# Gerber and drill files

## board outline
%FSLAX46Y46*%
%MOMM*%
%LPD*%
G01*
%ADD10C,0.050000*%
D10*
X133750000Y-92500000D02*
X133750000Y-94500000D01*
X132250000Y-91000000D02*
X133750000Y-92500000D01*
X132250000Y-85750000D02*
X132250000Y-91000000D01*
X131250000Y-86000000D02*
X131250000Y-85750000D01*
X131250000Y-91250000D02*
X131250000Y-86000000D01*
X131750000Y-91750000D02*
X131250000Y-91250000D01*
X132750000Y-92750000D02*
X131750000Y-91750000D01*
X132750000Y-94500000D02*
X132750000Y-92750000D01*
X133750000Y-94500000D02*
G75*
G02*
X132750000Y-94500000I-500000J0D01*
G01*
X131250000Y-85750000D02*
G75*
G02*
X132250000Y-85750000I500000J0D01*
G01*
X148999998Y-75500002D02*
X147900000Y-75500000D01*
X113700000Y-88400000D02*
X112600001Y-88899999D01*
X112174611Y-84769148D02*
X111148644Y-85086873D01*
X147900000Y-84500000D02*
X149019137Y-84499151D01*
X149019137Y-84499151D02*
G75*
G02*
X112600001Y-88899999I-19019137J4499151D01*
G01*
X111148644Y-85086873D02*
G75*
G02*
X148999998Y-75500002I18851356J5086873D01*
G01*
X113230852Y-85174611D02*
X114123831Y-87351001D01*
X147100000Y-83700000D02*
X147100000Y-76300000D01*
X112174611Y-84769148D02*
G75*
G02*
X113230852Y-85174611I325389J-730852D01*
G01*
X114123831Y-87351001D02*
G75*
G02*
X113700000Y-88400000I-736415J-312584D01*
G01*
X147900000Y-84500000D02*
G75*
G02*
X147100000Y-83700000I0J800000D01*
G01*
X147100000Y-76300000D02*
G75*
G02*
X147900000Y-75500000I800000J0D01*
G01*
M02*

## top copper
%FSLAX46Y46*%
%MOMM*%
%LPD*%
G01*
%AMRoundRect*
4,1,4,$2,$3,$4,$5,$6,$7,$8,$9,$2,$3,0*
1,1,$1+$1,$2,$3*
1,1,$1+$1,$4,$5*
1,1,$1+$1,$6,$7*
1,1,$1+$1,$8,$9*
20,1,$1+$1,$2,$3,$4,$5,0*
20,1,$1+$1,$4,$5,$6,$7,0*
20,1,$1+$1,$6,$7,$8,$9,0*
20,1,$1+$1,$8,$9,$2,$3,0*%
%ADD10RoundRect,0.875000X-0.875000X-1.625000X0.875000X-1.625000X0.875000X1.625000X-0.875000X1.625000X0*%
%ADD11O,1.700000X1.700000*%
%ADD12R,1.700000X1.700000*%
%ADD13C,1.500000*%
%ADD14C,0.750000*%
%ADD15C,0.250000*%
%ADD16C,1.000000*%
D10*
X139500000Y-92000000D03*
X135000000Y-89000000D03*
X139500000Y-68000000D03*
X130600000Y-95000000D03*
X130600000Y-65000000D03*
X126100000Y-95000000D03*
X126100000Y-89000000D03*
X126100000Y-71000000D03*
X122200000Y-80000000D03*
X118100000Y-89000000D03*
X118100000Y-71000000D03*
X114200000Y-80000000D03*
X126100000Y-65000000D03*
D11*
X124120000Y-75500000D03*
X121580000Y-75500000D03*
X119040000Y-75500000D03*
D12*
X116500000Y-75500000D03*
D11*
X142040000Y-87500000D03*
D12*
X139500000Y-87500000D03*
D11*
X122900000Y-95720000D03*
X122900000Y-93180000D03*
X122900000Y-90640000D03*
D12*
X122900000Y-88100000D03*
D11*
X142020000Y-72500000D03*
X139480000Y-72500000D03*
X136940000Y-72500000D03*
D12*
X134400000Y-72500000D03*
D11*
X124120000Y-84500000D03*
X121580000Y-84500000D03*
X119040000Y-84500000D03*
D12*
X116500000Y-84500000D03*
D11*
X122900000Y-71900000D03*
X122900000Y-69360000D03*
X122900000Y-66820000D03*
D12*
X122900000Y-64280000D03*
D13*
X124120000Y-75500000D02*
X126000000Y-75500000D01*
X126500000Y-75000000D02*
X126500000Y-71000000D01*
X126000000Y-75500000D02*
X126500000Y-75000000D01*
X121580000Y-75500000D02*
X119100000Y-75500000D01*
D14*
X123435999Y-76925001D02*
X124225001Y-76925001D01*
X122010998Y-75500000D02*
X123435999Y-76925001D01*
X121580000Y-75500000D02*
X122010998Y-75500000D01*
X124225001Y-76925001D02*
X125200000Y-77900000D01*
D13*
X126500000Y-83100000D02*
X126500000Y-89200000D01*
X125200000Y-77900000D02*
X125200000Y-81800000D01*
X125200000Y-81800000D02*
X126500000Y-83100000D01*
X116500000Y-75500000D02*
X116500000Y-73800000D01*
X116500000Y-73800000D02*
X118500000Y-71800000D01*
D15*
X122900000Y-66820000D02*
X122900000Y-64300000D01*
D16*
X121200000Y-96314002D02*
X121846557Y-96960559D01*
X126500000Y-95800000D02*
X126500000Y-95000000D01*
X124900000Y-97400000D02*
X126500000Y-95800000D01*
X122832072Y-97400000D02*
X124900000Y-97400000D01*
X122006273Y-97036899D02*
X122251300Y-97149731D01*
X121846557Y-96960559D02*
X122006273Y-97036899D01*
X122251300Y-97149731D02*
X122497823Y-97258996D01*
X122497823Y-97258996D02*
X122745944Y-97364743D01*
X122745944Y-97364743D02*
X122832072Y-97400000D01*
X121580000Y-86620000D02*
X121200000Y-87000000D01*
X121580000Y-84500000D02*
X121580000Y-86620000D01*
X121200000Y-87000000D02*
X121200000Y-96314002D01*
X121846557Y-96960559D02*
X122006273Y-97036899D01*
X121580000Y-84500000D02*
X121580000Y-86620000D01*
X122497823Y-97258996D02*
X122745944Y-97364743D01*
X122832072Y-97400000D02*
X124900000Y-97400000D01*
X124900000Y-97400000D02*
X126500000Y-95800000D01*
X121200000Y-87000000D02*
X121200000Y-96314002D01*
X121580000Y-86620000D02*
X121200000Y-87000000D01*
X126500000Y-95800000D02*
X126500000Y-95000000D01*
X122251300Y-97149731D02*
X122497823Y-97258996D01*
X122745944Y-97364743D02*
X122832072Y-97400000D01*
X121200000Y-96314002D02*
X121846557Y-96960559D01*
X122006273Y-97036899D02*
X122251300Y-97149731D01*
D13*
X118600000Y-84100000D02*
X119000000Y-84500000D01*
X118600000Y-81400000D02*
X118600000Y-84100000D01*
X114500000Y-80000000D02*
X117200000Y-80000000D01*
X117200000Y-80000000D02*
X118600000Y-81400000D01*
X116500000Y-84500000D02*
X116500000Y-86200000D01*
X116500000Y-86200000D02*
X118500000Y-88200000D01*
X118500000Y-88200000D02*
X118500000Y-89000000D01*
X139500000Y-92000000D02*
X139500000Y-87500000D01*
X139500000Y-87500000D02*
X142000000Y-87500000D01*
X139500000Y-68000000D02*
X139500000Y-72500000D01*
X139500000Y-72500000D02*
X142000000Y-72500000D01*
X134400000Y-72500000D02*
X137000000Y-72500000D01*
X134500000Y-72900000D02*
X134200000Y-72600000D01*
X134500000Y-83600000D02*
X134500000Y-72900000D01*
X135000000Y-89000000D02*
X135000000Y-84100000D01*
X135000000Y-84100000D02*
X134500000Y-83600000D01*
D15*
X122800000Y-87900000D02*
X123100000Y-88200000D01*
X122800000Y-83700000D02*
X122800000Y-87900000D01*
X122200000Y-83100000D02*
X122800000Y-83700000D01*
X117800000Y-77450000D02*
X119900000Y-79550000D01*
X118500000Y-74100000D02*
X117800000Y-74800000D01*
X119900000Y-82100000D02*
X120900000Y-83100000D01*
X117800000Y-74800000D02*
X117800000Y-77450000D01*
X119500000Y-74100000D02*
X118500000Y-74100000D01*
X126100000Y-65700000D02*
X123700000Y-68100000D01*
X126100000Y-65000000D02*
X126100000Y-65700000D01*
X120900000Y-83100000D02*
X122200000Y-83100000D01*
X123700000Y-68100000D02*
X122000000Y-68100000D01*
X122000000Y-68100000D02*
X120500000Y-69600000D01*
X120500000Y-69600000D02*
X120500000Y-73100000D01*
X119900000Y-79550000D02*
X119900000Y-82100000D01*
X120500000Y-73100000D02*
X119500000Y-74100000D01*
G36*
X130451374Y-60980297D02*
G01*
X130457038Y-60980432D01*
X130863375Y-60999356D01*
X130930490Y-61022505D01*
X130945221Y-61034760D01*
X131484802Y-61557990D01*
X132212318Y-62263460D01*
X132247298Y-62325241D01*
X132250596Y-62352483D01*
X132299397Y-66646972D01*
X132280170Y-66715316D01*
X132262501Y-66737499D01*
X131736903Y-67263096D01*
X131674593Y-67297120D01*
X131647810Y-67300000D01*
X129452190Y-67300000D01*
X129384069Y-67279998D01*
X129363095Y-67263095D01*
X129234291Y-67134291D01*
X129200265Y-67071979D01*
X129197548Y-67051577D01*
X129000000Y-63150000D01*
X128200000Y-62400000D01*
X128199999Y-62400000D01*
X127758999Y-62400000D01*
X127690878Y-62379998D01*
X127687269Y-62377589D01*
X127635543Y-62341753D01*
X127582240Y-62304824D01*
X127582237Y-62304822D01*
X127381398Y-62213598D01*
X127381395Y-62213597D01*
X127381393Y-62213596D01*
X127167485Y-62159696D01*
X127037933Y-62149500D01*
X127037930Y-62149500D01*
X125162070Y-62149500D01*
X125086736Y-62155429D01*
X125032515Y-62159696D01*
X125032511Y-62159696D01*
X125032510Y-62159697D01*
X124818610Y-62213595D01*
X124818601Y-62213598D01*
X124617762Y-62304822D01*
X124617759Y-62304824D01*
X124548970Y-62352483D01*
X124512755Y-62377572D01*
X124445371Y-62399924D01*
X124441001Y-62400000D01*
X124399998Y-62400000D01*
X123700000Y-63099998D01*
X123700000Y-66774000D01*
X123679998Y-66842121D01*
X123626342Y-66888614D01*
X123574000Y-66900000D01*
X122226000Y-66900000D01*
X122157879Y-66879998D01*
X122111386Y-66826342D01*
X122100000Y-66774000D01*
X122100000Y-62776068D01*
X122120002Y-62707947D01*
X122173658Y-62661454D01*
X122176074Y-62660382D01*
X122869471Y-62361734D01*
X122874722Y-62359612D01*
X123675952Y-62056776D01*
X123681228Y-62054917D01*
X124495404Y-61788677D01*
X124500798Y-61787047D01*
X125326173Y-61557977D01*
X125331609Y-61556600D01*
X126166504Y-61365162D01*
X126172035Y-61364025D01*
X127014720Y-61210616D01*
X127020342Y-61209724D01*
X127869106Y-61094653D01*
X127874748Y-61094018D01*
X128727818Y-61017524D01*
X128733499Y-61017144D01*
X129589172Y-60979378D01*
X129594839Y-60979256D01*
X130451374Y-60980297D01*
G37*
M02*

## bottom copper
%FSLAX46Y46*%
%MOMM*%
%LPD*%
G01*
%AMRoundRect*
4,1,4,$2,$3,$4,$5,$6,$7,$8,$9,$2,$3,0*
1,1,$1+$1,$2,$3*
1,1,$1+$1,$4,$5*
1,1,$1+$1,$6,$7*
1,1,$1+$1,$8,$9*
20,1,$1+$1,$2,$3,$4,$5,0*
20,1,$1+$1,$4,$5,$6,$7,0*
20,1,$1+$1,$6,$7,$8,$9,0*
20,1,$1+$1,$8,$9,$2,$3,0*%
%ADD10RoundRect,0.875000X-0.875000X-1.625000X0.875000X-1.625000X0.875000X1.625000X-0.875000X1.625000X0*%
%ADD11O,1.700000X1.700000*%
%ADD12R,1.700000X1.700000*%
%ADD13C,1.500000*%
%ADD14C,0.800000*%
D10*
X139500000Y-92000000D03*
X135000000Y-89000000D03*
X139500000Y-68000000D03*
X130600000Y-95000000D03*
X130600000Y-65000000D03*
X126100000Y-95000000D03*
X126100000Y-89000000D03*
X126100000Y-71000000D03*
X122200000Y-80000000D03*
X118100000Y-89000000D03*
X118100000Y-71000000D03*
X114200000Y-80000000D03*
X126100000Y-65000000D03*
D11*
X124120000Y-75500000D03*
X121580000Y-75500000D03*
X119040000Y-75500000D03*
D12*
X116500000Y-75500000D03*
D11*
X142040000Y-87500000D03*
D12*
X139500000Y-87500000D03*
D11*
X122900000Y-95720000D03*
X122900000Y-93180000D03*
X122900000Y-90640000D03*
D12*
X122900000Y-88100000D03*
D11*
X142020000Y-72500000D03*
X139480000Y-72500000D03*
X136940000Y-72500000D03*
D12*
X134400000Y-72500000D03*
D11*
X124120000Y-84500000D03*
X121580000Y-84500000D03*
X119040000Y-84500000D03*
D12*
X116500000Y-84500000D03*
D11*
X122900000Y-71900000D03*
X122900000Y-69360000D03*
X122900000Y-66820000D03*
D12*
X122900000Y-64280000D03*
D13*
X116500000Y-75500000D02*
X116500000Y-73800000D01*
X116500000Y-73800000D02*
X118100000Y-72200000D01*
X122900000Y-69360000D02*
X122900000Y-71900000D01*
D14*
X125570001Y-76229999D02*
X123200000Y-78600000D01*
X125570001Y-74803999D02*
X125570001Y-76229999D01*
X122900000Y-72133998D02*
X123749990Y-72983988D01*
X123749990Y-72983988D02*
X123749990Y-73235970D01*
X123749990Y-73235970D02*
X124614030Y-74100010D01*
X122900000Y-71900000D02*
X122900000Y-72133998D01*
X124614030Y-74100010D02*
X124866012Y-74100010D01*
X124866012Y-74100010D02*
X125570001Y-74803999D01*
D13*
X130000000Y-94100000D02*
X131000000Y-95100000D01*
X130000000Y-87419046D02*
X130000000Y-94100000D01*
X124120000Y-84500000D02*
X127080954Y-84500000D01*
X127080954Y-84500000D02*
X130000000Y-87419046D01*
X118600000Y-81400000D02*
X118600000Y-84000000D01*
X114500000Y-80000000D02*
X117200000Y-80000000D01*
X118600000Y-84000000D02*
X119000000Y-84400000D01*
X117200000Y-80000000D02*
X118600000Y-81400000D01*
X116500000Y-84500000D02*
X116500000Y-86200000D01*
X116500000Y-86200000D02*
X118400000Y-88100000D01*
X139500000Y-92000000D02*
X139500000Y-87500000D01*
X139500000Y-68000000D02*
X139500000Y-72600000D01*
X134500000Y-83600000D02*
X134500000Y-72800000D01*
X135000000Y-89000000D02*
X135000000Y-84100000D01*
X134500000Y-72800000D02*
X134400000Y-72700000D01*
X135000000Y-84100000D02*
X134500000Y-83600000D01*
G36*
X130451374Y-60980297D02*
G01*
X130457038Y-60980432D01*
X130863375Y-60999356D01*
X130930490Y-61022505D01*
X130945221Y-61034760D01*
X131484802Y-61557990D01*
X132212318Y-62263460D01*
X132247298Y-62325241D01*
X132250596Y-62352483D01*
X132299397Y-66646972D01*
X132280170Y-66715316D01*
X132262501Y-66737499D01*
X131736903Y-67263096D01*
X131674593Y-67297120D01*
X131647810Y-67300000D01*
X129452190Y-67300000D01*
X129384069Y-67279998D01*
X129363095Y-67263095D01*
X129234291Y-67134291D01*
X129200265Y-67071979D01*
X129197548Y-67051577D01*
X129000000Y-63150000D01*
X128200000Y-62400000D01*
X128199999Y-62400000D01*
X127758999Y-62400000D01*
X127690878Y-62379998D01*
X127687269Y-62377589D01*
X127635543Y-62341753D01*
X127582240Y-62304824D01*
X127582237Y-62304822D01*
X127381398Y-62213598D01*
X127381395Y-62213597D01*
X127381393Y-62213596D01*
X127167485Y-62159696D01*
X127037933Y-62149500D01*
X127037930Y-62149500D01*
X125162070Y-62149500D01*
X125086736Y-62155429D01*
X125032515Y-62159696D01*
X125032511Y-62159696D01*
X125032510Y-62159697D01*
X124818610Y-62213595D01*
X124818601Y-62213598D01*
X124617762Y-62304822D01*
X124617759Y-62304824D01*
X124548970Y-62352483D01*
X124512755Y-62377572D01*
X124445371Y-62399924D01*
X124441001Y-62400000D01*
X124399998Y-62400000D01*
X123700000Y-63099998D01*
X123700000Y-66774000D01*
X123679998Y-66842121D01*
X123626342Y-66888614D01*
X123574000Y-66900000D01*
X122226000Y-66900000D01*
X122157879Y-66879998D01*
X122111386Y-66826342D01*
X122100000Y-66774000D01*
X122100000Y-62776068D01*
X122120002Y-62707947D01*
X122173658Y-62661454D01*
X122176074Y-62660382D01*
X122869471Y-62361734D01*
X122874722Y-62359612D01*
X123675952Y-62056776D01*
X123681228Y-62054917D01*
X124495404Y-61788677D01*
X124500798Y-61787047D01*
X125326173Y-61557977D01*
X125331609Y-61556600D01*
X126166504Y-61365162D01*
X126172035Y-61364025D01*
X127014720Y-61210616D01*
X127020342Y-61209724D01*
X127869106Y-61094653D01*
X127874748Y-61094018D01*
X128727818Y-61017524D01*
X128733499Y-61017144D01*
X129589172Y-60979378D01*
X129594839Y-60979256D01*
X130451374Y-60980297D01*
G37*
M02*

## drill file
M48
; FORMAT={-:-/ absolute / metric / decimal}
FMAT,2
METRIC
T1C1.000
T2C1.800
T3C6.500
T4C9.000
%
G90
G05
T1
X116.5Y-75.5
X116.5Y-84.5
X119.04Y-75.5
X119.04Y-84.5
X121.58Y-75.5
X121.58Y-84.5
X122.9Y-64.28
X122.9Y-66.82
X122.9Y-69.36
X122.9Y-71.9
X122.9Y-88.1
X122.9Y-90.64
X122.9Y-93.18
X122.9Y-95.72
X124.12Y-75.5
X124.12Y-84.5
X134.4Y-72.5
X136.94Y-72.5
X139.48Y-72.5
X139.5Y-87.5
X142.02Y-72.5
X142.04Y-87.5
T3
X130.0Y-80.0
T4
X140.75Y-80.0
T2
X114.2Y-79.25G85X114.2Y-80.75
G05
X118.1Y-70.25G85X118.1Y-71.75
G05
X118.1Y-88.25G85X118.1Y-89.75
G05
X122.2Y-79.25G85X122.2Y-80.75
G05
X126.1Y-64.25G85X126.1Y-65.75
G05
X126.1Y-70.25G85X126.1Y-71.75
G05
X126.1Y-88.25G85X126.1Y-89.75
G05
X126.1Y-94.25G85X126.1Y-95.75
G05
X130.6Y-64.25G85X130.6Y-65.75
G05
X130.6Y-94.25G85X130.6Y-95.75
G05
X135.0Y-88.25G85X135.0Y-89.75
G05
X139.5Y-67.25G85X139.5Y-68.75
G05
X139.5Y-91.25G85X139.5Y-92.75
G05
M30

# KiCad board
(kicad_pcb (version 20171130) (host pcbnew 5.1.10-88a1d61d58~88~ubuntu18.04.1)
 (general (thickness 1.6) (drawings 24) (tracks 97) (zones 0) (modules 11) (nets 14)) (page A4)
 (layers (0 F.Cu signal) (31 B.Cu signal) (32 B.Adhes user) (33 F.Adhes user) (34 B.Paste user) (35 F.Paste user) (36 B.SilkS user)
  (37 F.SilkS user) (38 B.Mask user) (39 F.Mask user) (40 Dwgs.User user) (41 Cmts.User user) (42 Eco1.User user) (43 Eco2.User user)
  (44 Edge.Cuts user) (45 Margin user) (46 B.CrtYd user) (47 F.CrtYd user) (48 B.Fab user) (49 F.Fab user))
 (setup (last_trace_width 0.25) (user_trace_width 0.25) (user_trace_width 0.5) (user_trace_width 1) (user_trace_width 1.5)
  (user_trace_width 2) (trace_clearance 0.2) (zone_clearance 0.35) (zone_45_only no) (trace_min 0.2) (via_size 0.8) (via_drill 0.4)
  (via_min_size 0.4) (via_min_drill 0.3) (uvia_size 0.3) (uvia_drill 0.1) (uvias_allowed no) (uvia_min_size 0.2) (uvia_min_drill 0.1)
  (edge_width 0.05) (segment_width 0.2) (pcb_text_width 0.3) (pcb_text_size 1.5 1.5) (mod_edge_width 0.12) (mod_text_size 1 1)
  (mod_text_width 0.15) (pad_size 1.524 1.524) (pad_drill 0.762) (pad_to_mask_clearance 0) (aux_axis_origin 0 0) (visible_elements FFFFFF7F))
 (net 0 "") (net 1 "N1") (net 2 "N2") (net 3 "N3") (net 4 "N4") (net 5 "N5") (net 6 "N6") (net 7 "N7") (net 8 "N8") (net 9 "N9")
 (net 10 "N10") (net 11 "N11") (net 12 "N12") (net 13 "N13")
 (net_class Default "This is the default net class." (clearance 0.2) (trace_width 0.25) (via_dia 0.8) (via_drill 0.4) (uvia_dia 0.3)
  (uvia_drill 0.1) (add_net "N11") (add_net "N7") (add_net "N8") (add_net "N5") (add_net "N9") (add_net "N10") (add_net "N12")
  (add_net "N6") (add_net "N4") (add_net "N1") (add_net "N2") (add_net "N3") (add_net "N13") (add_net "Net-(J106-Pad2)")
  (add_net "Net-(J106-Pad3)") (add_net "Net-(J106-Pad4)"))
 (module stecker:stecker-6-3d (layer F.Cu) (at 130 80)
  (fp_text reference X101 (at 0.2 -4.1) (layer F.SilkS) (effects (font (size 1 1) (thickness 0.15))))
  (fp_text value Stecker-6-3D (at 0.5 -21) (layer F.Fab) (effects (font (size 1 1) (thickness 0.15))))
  (pad 24 thru_hole roundrect (at 9.5 12) (size 3.5 5) (drill oval 1.8 3.3) (layers *.Cu *.Mask) (roundrect_rratio 0.25) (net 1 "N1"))
  (pad 21 thru_hole roundrect (at 5 9) (size 3.5 5) (drill oval 1.8 3.3) (layers *.Cu *.Mask) (roundrect_rratio 0.25) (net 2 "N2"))
  (pad 23 thru_hole roundrect (at 9.5 -12) (size 3.5 5) (drill oval 1.8 3.3) (layers *.Cu *.Mask) (roundrect_rratio 0.25) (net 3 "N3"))
  (pad 18 thru_hole roundrect (at 0.6 15) (size 3.5 5) (drill oval 1.8 3.3) (layers *.Cu *.Mask) (roundrect_rratio 0.25) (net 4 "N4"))
  (pad 15 thru_hole roundrect (at 0.6 -15) (size 3.5 5) (drill oval 1.8 3.3) (layers *.Cu *.Mask) (roundrect_rratio 0.25) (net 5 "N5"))
  (pad 14 thru_hole roundrect (at -3.9 15) (size 3.5 5) (drill oval 1.8 3.3) (layers *.Cu *.Mask) (roundrect_rratio 0.25) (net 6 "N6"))
  (pad 13 thru_hole roundrect (at -3.9 9) (size 3.5 5) (drill oval 1.8 3.3) (layers *.Cu *.Mask) (roundrect_rratio 0.25) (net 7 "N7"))
  (pad 12 thru_hole roundrect (at -3.9 -9) (size 3.5 5) (drill oval 1.8 3.3) (layers *.Cu *.Mask) (roundrect_rratio 0.25) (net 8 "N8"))
  (pad 8 thru_hole roundrect (at -7.8 0) (size 3.5 5) (drill oval 1.8 3.3) (layers *.Cu *.Mask) (roundrect_rratio 0.25) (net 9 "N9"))
  (pad 5 thru_hole roundrect (at -11.9 9) (size 3.5 5) (drill oval 1.8 3.3) (layers *.Cu *.Mask) (roundrect_rratio 0.25) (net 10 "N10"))
  (pad 2 thru_hole roundrect (at -11.9 -9) (size 3.5 5) (drill oval 1.8 3.3) (layers *.Cu *.Mask) (roundrect_rratio 0.25) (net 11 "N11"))
  (pad 1 thru_hole roundrect (at -15.8 0) (size 3.5 5) (drill oval 1.8 3.3) (layers *.Cu *.Mask) (roundrect_rratio 0.25) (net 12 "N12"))
  (pad "" np_thru_hole circle (at 10.75 0) (size 9 9) (drill 9) (layers *.Cu *.Mask))
  (pad "" np_thru_hole circle (at 0 0) (size 6.5 6.5) (drill 6.5) (layers *.Cu *.Mask))
  (pad 11 thru_hole roundrect (at -3.9 -15) (size 3.5 5) (drill oval 1.8 3.3) (layers *.Cu *.Mask) (roundrect_rratio 0.25) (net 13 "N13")))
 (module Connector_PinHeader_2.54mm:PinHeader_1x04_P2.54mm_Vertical (layer F.Cu) (at 116.5 75.5 90)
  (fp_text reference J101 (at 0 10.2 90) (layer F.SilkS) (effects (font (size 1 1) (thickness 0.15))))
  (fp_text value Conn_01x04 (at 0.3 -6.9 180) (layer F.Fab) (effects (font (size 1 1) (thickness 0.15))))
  (pad 4 thru_hole oval (at 0 7.62 90) (size 1.7 1.7) (drill 1) (layers *.Cu *.Mask) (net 8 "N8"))
  (pad 3 thru_hole oval (at 0 5.08 90) (size 1.7 1.7) (drill 1) (layers *.Cu *.Mask) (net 7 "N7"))
  (pad 2 thru_hole oval (at 0 2.54 90) (size 1.7 1.7) (drill 1) (layers *.Cu *.Mask) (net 7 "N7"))
  (pad 1 thru_hole rect (at 0 0 90) (size 1.7 1.7) (drill 1) (layers *.Cu *.Mask) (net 11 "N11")))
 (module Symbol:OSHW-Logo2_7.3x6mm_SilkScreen (layer F.Cu) (at 135.4 64.5 270)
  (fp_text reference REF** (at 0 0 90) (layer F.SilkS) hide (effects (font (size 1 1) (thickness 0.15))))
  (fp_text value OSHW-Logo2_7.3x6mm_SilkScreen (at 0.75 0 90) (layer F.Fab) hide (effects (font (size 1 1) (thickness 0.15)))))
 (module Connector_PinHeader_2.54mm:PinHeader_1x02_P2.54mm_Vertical (layer F.Cu) (at 139.5 87.5 90)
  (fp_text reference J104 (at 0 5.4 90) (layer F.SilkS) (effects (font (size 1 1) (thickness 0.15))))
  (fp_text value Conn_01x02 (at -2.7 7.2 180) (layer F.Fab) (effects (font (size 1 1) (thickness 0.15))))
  (pad 2 thru_hole oval (at 0 2.54 90) (size 1.7 1.7) (drill 1) (layers *.Cu *.Mask) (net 1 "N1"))
  (pad 1 thru_hole rect (at 0 0 90) (size 1.7 1.7) (drill 1) (layers *.Cu *.Mask) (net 1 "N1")))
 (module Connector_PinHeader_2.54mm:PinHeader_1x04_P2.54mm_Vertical (layer F.Cu) (at 122.9 88.1)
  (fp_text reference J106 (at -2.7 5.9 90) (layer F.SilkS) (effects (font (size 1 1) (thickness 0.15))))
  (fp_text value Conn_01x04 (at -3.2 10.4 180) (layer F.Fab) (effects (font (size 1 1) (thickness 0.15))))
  (pad 4 thru_hole oval (at 0 7.62) (size 1.7 1.7) (drill 1) (layers *.Cu *.Mask))
  (pad 3 thru_hole oval (at 0 5.08) (size 1.7 1.7) (drill 1) (layers *.Cu *.Mask))
  (pad 2 thru_hole oval (at 0 2.54) (size 1.7 1.7) (drill 1) (layers *.Cu *.Mask))
  (pad 1 thru_hole rect (at 0 0) (size 1.7 1.7) (drill 1) (layers *.Cu *.Mask) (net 13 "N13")))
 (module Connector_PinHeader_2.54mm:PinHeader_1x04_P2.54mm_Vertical (layer F.Cu) (at 134.4 72.5 90)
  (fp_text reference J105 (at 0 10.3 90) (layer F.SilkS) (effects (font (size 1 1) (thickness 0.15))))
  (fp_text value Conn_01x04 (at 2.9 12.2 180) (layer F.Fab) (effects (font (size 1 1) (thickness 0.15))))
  (pad 4 thru_hole oval (at 0 7.62 90) (size 1.7 1.7) (drill 1) (layers *.Cu *.Mask) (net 3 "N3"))
  (pad 3 thru_hole oval (at 0 5.08 90) (size 1.7 1.7) (drill 1) (layers *.Cu *.Mask) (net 3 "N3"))
  (pad 2 thru_hole oval (at 0 2.54 90) (size 1.7 1.7) (drill 1) (layers *.Cu *.Mask) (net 2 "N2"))
  (pad 1 thru_hole rect (at 0 0 90) (size 1.7 1.7) (drill 1) (layers *.Cu *.Mask) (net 2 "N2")))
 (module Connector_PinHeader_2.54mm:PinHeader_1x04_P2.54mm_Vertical (layer F.Cu) (at 116.5 84.5 90)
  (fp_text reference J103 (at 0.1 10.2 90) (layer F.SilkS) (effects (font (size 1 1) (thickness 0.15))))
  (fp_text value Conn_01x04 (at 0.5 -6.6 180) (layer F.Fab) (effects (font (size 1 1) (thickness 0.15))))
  (pad 4 thru_hole oval (at 0 7.62 90) (size 1.7 1.7) (drill 1) (layers *.Cu *.Mask) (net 4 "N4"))
  (pad 3 thru_hole oval (at 0 5.08 90) (size 1.7 1.7) (drill 1) (layers *.Cu *.Mask) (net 6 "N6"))
  (pad 2 thru_hole oval (at 0 2.54 90) (size 1.7 1.7) (drill 1) (layers *.Cu *.Mask) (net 12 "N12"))
  (pad 1 thru_hole rect (at 0 0 90) (size 1.7 1.7) (drill 1) (layers *.Cu *.Mask) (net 10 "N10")))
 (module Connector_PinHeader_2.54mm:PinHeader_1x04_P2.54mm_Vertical (layer F.Cu) (at 122.9 64.28)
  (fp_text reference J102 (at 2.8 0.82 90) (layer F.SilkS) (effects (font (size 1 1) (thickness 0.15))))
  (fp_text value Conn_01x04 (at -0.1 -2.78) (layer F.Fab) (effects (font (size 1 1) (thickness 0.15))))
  (pad 4 thru_hole oval (at 0 7.62) (size 1.7 1.7) (drill 1) (layers *.Cu *.Mask) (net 9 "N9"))
  (pad 3 thru_hole oval (at 0 5.08) (size 1.7 1.7) (drill 1) (layers *.Cu *.Mask) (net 9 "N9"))
  (pad 2 thru_hole oval (at 0 2.54) (size 1.7 1.7) (drill 1) (layers *.Cu *.Mask) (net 5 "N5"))
  (pad 1 thru_hole rect (at 0 0) (size 1.7 1.7) (drill 1) (layers *.Cu *.Mask) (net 5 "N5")))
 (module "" (layer F.Cu) (at -14.4 40.9)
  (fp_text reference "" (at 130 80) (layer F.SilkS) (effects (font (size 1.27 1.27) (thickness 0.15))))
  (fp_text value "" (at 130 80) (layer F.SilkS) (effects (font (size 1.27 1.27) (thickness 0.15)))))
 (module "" (layer F.Cu) (at -16.3 40)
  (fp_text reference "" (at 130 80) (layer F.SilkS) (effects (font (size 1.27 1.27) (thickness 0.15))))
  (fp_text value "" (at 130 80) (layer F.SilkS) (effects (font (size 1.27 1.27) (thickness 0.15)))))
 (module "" (layer F.Cu) (at -13.8 35.7)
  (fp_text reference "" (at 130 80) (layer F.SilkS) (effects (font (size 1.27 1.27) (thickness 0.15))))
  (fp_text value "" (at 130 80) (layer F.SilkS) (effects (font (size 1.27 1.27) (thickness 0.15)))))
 (gr_line (start 133.75 92.5) (end 133.75 94.5) (layer Edge.Cuts) (width 0.05))
 (gr_line (start 132.25 91) (end 133.75 92.5) (layer Edge.Cuts) (width 0.05))
 (gr_line (start 132.25 85.75) (end 132.25 91) (layer Edge.Cuts) (width 0.05))
 (gr_line (start 131.25 86) (end 131.25 85.75) (layer Edge.Cuts) (width 0.05))
 (gr_line (start 131.25 91.25) (end 131.25 86) (layer Edge.Cuts) (width 0.05))
 (gr_line (start 131.75 91.75) (end 131.25 91.25) (layer Edge.Cuts) (width 0.05))
 (gr_line (start 132.75 92.75) (end 131.75 91.75) (layer Edge.Cuts) (width 0.05))
 (gr_line (start 132.75 94.5) (end 132.75 92.75) (layer Edge.Cuts) (width 0.05))
 (gr_arc (start 133.25 94.5) (end 132.75 94.5) (angle -180) (layer Edge.Cuts) (width 0.05))
 (gr_arc (start 131.75 85.75) (end 132.25 85.75) (angle -180) (layer Edge.Cuts) (width 0.05))
 (gr_line (start 148.999998 75.500002) (end 147.9 75.5) (layer Edge.Cuts) (width 0.05))
 (gr_line (start 113.7 88.4) (end 112.600001 88.899999) (layer Edge.Cuts) (width 0.05))
 (gr_line (start 112.174611 84.769148) (end 111.148644 85.086873) (layer Edge.Cuts) (width 0.05))
 (gr_line (start 147.9 84.5) (end 149.019137 84.499151) (layer Edge.Cuts) (width 0.05))
 (gr_arc (start 130 80) (end 112.600001 88.899999) (angle -139.6013383) (layer Edge.Cuts) (width 0.05))
 (gr_arc (start 130 80) (end 148.999998 75.500002) (angle -181.7765691) (layer Edge.Cuts) (width 0.05))
 (gr_line (start 113.230852 85.174611) (end 114.123831 87.351001) (layer Edge.Cuts) (width 0.05))
 (gr_line (start 147.1 83.7) (end 147.1 76.3) (layer Edge.Cuts) (width 0.05))
 (gr_arc (start 112.5 85.5) (end 113.230852 85.174611) (angle -90) (layer Edge.Cuts) (width 0.05))
 (gr_arc (start 113.387416 87.663585) (end 113.7 88.4) (angle -90) (layer Edge.Cuts) (width 0.05))
 (gr_arc (start 147.9 83.7) (end 147.1 83.7) (angle -90) (layer Edge.Cuts) (width 0.05))
 (gr_arc (start 147.9 76.3) (end 147.9 75.5) (angle -90) (layer Edge.Cuts) (width 0.05))
 (segment (start 124.12 75.5) (end 126 75.5) (width 1.5) (layer F.Cu) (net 8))
 (segment (start 126.5 75) (end 126.5 71) (width 1.5) (layer F.Cu) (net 8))
 (segment (start 126 75.5) (end 126.5 75) (width 1.5) (layer F.Cu) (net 8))
 (segment (start 121.58 75.5) (end 119.1 75.5) (width 1.5) (layer F.Cu) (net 7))
 (segment (start 123.435999 76.925001) (end 124.225001 76.925001) (width 0.75) (layer F.Cu) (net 7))
 (segment (start 122.010998 75.5) (end 123.435999 76.925001) (width 0.75) (layer F.Cu) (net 7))
 (segment (start 121.58 75.5) (end 122.010998 75.5) (width 0.75) (layer F.Cu) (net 7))
 (segment (start 124.225001 76.925001) (end 125.2 77.9) (width 0.75) (layer F.Cu) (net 7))
 (segment (start 126.5 83.1) (end 126.5 89.2) (width 1.5) (layer F.Cu) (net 7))
 (segment (start 125.2 77.9) (end 125.2 81.8) (width 1.5) (layer F.Cu) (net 7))
 (segment (start 125.2 81.8) (end 126.5 83.1) (width 1.5) (layer F.Cu) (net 7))
 (segment (start 116.5 75.5) (end 116.5 73.8) (width 1.5) (layer F.Cu) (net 11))
 (segment (start 116.5 73.8) (end 118.5 71.8) (width 1.5) (layer F.Cu) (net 11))
 (segment (start 116.5 75.5) (end 116.5 73.8) (width 1.5) (layer B.Cu) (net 11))
 (segment (start 116.5 73.8) (end 118.1 72.2) (width 1.5) (layer B.Cu) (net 11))
 (segment (start 122.9 69.36) (end 122.9 71.9) (width 1.5) (layer B.Cu) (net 9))
 (segment (start 125.570001 76.229999) (end 123.2 78.6) (width 0.8) (layer B.Cu) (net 9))
 (segment (start 125.570001 74.803999) (end 125.570001 76.229999) (width 0.8) (layer B.Cu) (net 9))
 (segment (start 122.9 72.133998) (end 123.74999 72.983988) (width 0.8) (layer B.Cu) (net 9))
 (segment (start 123.74999 72.983988) (end 123.74999 73.23597) (width 0.8) (layer B.Cu) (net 9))
 (segment (start 123.74999 73.23597) (end 124.61403 74.10001) (width 0.8) (layer B.Cu) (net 9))
 (segment (start 122.9 71.9) (end 122.9 72.133998) (width 0.8) (layer B.Cu) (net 9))
 (segment (start 124.61403 74.10001) (end 124.866012 74.10001) (width 0.8) (layer B.Cu) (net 9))
 (segment (start 124.866012 74.10001) (end 125.570001 74.803999) (width 0.8) (layer B.Cu) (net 9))
 (segment (start 122.9 66.82) (end 122.9 64.3) (width 0.25) (layer F.Cu) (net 5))
 (segment (start 130 94.1) (end 131 95.1) (width 1.5) (layer B.Cu) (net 4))
 (segment (start 130 87.419046) (end 130 94.1) (width 1.5) (layer B.Cu) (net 4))
 (segment (start 124.12 84.5) (end 127.080954 84.5) (width 1.5) (layer B.Cu) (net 4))
 (segment (start 127.080954 84.5) (end 130 87.419046) (width 1.5) (layer B.Cu) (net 4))
 (segment (start 121.2 96.314002) (end 121.846557 96.960559) (width 1) (layer F.Cu) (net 6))
 (segment (start 126.5 95.8) (end 126.5 95) (width 1) (layer F.Cu) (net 6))
 (segment (start 124.9 97.4) (end 126.5 95.8) (width 1) (layer F.Cu) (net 6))
 (segment (start 122.832072 97.4) (end 124.9 97.4) (width 1) (layer F.Cu) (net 6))
 (segment (start 122.006273 97.036899) (end 122.2513 97.149731) (width 1) (layer F.Cu) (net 6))
 (segment (start 121.846557 96.960559) (end 122.006273 97.036899) (width 1) (layer F.Cu) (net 6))
 (segment (start 122.2513 97.149731) (end 122.497823 97.258996) (width 1) (layer F.Cu) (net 6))
 (segment (start 122.497823 97.258996) (end 122.745944 97.364743) (width 1) (layer F.Cu) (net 6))
 (segment (start 122.745944 97.364743) (end 122.832072 97.4) (width 1) (layer F.Cu) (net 6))
 (segment (start 121.58 86.62) (end 121.2 87) (width 1) (layer F.Cu) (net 6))
 (segment (start 121.58 84.5) (end 121.58 86.62) (width 1) (layer F.Cu) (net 6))
 (segment (start 121.2 87) (end 121.2 96.314002) (width 1) (layer F.Cu) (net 6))
 (segment (start 121.846557 96.960559) (end 122.006273 97.036899) (width 1) (layer F.Cu) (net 6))
 (segment (start 121.58 84.5) (end 121.58 86.62) (width 1) (layer F.Cu) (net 6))
 (segment (start 122.497823 97.258996) (end 122.745944 97.364743) (width 1) (layer F.Cu) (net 6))
 (segment (start 122.832072 97.4) (end 124.9 97.4) (width 1) (layer F.Cu) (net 6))
 (segment (start 124.9 97.4) (end 126.5 95.8) (width 1) (layer F.Cu) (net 6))
 (segment (start 121.2 87) (end 121.2 96.314002) (width 1) (layer F.Cu) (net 6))
 (segment (start 121.58 86.62) (end 121.2 87) (width 1) (layer F.Cu) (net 6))
 (segment (start 126.5 95.8) (end 126.5 95) (width 1) (layer F.Cu) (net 6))
 (segment (start 122.2513 97.149731) (end 122.497823 97.258996) (width 1) (layer F.Cu) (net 6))
 (segment (start 122.745944 97.364743) (end 122.832072 97.4) (width 1) (layer F.Cu) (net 6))
 (segment (start 121.2 96.314002) (end 121.846557 96.960559) (width 1) (layer F.Cu) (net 6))
 (segment (start 122.006273 97.036899) (end 122.2513 97.149731) (width 1) (layer F.Cu) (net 6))
 (segment (start 118.6 84.1) (end 119 84.5) (width 1.5) (layer F.Cu) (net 12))
 (segment (start 118.6 81.4) (end 118.6 84.1) (width 1.5) (layer F.Cu) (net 12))
 (segment (start 114.5 80) (end 117.2 80) (width 1.5) (layer F.Cu) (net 12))
 (segment (start 117.2 80) (end 118.6 81.4) (width 1.5) (layer F.Cu) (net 12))
 (segment (start 118.6 81.4) (end 118.6 84) (width 1.5) (layer B.Cu) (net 12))
 (segment (start 114.5 80) (end 117.2 80) (width 1.5) (layer B.Cu) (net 12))
 (segment (start 118.6 84) (end 119 84.4) (width 1.5) (layer B.Cu) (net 12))
 (segment (start 117.2 80) (end 118.6 81.4) (width 1.5) (layer B.Cu) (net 12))
 (segment (start 116.5 84.5) (end 116.5 86.2) (width 1.5) (layer F.Cu) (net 10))
 (segment (start 116.5 86.2) (end 118.5 88.2) (width 1.5) (layer F.Cu) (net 10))
 (segment (start 118.5 88.2) (end 118.5 89) (width 1.5) (layer F.Cu) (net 10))
 (segment (start 116.5 84.5) (end 116.5 86.2) (width 1.5) (layer B.Cu) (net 10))
 (segment (start 116.5 86.2) (end 118.4 88.1) (width 1.5) (layer B.Cu) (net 10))
 (segment (start 139.5 92) (end 139.5 87.5) (width 1.5) (layer F.Cu) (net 1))
 (segment (start 139.5 87.5) (end 142 87.5) (width 1.5) (layer F.Cu) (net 1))
 (segment (start 139.5 92) (end 139.5 87.5) (width 1.5) (layer B.Cu) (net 1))
 (segment (start 139.5 68) (end 139.5 72.5) (width 1.5) (layer F.Cu) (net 3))
 (segment (start 139.5 72.5) (end 142 72.5) (width 1.5) (layer F.Cu) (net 3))
 (segment (start 139.5 68) (end 139.5 72.6) (width 1.5) (layer B.Cu) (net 3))
 (segment (start 134.4 72.5) (end 137 72.5) (width 1.5) (layer F.Cu) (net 2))
 (segment (start 134.5 72.9) (end 134.2 72.6) (width 1.5) (layer F.Cu) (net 2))
 (segment (start 134.5 83.6) (end 134.5 72.9) (width 1.5) (layer F.Cu) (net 2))
 (segment (start 135 89) (end 135 84.1) (width 1.5) (layer F.Cu) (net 2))
 (segment (start 135 84.1) (end 134.5 83.6) (width 1.5) (layer F.Cu) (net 2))
 (segment (start 134.5 83.6) (end 134.5 72.8) (width 1.5) (layer B.Cu) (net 2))
 (segment (start 135 89) (end 135 84.1) (width 1.5) (layer B.Cu) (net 2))
 (segment (start 134.5 72.8) (end 134.4 72.7) (width 1.5) (layer B.Cu) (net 2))
 (segment (start 135 84.1) (end 134.5 83.6) (width 1.5) (layer B.Cu) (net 2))
 (segment (start 122.8 87.9) (end 123.1 88.2) (width 0.25) (layer F.Cu) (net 13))
 (segment (start 122.8 83.7) (end 122.8 87.9) (width 0.25) (layer F.Cu) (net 13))
 (segment (start 122.2 83.1) (end 122.8 83.7) (width 0.25) (layer F.Cu) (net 13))
 (segment (start 117.8 77.45) (end 119.9 79.55) (width 0.25) (layer F.Cu) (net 13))
 (segment (start 118.5 74.1) (end 117.8 74.8) (width 0.25) (layer F.Cu) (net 13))
 (segment (start 119.9 82.1) (end 120.9 83.1) (width 0.25) (layer F.Cu) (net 13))
 (segment (start 117.8 74.8) (end 117.8 77.45) (width 0.25) (layer F.Cu) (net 13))
 (segment (start 119.5 74.1) (end 118.5 74.1) (width 0.25) (layer F.Cu) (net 13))
 (segment (start 126.1 65.7) (end 123.7 68.1) (width 0.25) (layer F.Cu) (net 13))
 (segment (start 126.1 65) (end 126.1 65.7) (width 0.25) (layer F.Cu) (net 13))
 (segment (start 120.9 83.1) (end 122.2 83.1) (width 0.25) (layer F.Cu) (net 13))
 (segment (start 123.7 68.1) (end 122 68.1) (width 0.25) (layer F.Cu) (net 13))
 (segment (start 122 68.1) (end 120.5 69.6) (width 0.25) (layer F.Cu) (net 13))
 (segment (start 120.5 69.6) (end 120.5 73.1) (width 0.25) (layer F.Cu) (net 13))
 (segment (start 119.9 79.55) (end 119.9 82.1) (width 0.25) (layer F.Cu) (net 13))
 (segment (start 120.5 73.1) (end 119.5 74.1) (width 0.25) (layer F.Cu) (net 13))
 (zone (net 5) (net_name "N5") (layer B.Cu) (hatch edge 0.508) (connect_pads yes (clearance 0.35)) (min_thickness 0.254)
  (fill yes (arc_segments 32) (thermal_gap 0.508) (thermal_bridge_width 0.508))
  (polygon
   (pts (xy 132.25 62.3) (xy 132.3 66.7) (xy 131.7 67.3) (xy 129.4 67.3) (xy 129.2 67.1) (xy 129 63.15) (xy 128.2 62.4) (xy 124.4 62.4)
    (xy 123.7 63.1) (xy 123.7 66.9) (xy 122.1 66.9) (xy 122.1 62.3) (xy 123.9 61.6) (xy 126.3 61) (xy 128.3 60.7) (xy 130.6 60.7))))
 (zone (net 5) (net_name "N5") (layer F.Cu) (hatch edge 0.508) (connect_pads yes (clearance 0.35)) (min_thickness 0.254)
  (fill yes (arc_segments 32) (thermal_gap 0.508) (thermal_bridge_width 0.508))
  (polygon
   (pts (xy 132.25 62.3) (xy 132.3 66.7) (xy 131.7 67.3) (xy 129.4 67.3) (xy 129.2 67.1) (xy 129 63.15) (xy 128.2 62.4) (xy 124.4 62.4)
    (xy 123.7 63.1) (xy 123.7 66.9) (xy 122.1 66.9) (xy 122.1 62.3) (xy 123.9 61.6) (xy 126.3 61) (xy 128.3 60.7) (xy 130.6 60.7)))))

